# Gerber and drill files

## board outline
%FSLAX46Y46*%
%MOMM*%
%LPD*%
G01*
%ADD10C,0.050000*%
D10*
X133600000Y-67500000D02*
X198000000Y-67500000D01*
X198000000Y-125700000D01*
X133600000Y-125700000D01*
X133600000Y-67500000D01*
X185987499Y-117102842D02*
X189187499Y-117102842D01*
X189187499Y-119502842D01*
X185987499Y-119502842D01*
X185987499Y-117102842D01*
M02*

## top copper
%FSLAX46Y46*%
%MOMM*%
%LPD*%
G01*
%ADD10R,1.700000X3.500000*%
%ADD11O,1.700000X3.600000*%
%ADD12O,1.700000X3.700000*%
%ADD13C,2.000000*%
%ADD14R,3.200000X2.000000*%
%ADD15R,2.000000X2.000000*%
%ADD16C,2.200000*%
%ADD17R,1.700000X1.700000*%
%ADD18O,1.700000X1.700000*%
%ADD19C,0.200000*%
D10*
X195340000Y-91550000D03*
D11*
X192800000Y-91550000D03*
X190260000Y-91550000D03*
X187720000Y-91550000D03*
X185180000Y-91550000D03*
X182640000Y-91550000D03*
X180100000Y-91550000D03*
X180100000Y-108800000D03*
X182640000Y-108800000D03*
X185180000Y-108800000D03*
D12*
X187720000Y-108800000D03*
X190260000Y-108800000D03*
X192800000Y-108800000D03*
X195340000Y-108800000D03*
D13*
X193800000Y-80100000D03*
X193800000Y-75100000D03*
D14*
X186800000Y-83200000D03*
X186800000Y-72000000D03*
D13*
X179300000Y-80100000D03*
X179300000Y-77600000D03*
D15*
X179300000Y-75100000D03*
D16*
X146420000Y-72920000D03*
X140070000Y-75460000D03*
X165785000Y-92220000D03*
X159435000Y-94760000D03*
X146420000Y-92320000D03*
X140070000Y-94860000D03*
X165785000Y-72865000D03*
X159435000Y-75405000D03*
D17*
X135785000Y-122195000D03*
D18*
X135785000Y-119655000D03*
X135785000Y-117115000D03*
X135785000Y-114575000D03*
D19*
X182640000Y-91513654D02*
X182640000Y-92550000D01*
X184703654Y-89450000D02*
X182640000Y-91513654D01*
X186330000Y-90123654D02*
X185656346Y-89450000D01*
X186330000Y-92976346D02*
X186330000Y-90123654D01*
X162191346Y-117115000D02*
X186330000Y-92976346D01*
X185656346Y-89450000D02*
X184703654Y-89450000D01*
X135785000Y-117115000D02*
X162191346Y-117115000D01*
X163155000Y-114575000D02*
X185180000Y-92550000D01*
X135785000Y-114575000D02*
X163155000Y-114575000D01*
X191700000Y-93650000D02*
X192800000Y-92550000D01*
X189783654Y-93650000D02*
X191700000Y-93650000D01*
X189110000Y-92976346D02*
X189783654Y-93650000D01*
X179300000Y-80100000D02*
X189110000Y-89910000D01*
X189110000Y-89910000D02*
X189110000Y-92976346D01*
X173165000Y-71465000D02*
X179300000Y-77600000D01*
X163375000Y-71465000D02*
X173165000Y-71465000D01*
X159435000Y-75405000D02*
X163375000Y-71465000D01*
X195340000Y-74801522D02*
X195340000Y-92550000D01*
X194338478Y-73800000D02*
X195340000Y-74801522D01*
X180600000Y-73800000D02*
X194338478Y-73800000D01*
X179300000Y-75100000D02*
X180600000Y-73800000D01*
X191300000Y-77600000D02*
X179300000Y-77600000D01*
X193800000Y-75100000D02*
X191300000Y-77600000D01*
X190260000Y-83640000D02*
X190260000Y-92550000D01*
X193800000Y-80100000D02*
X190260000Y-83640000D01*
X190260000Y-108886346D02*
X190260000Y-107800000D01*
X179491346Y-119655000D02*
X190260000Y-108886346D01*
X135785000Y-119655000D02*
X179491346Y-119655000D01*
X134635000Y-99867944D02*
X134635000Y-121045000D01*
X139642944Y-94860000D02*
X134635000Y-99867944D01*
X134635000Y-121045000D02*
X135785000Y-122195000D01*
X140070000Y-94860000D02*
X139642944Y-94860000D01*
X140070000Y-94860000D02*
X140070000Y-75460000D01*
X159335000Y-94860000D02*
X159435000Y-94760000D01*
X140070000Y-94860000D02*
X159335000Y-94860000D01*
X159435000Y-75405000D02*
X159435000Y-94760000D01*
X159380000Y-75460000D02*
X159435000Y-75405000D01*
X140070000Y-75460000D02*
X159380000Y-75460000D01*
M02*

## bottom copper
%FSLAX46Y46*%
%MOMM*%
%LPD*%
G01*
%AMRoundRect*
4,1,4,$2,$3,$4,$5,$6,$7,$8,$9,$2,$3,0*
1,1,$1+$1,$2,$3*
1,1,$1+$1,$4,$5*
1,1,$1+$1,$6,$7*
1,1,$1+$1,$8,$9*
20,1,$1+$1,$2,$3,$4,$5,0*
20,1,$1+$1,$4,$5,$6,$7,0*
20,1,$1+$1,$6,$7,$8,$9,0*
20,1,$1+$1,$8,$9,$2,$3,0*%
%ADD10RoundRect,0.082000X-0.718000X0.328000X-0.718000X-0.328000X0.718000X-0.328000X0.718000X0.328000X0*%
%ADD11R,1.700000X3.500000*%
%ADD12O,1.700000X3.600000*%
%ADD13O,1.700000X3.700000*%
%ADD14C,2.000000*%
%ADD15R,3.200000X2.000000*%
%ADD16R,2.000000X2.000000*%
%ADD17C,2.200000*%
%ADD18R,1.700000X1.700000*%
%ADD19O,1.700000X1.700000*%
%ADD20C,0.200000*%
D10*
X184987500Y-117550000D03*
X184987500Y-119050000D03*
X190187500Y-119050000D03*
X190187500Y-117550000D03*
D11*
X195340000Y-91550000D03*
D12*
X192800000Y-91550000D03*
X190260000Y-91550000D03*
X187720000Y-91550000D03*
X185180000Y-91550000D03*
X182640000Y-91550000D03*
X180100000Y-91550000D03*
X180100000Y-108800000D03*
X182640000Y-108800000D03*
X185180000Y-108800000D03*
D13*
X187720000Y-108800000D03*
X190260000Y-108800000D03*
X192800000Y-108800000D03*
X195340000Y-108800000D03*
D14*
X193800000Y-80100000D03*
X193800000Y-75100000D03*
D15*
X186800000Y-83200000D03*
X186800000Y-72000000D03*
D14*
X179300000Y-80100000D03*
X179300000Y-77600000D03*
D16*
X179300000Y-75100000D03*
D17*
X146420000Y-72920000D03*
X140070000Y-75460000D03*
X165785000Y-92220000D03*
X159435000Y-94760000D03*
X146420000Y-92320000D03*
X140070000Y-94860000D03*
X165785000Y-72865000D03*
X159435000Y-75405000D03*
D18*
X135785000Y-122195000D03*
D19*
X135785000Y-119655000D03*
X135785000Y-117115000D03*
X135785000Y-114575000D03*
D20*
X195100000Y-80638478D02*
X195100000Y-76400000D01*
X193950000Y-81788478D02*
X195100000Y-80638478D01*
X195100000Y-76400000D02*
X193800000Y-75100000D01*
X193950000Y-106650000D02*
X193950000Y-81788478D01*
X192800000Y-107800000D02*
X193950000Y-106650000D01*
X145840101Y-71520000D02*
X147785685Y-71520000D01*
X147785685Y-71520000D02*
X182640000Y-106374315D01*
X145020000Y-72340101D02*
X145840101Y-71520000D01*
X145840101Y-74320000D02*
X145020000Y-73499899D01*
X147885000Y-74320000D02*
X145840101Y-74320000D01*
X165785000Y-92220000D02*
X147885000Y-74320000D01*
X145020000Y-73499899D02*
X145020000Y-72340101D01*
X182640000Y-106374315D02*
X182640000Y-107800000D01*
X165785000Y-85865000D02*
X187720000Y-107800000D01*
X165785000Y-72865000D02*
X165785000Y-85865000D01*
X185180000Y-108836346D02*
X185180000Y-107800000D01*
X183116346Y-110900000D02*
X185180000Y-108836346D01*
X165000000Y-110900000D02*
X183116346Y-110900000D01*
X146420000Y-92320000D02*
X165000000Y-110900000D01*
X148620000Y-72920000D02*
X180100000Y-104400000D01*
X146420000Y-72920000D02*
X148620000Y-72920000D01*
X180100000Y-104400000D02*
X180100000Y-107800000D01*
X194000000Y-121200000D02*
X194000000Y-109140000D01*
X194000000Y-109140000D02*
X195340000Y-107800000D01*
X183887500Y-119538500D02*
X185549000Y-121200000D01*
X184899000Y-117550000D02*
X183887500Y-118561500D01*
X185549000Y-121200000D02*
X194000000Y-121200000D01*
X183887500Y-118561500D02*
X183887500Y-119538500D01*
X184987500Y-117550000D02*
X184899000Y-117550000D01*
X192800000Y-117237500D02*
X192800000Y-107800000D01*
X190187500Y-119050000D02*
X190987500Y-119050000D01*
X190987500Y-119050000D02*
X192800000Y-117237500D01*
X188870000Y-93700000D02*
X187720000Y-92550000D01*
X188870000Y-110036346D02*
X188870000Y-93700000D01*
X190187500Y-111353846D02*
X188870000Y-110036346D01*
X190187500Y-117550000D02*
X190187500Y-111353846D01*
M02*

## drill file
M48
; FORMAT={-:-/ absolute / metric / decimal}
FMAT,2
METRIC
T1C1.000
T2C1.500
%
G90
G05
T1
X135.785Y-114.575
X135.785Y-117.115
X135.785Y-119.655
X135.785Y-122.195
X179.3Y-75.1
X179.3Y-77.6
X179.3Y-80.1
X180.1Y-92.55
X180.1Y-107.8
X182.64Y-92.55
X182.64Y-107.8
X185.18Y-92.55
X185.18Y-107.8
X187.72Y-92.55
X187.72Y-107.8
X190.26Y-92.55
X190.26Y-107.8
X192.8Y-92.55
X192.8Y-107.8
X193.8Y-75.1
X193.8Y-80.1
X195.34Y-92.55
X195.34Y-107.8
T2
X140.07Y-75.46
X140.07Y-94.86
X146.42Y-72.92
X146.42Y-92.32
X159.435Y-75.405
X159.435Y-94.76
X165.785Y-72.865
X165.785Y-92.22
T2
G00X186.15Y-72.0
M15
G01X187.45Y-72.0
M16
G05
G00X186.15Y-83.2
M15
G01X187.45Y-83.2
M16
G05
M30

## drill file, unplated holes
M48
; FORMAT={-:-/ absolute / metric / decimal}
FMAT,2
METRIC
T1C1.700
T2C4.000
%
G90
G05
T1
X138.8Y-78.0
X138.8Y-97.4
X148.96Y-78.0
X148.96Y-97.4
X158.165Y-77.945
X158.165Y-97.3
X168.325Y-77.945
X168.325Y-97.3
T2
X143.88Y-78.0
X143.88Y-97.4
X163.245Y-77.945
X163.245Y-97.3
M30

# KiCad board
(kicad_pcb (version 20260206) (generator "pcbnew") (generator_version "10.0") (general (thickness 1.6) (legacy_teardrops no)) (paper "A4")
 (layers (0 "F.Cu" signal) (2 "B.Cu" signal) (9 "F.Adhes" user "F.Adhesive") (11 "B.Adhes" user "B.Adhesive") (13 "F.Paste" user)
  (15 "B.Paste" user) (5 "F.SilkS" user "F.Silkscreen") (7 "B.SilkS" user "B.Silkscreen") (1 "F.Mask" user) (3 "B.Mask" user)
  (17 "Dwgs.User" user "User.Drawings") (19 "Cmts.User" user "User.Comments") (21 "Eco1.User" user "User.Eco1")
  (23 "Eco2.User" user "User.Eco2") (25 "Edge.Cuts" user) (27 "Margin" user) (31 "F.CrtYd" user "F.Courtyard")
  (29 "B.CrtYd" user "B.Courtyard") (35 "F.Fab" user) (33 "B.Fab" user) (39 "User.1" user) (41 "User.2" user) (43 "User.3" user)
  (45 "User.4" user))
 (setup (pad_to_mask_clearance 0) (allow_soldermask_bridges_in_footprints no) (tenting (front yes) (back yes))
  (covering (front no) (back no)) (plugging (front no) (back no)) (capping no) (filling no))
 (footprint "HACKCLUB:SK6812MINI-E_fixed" (layer "F.Cu") (at 187.587499 118.402842)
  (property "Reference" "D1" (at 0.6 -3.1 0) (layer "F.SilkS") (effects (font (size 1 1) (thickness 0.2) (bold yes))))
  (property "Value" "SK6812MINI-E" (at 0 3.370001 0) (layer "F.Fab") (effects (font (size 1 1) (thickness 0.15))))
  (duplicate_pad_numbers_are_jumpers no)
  (fp_rect (start -1.6 -1.3) (end 1.6 1.1) (stroke (width 0.05) (type default)) (fill no) (layer "Edge.Cuts"))
  (pad "1" smd roundrect (at -2.599999 -0.852842 270) (size 0.82 1.6) (layers "B.Cu" "B.Mask" "B.Paste") (roundrect_rratio 0.1)
   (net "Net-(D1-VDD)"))
  (pad "2" smd roundrect (at -2.599999 0.647158 270) (size 0.82 1.6) (layers "B.Cu" "B.Mask" "B.Paste") (roundrect_rratio 0.1)
   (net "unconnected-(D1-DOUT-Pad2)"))
  (pad "3" smd roundrect (at 2.600001 0.647158 270) (size 0.82 1.6) (layers "B.Cu" "B.Mask" "B.Paste") (roundrect_rratio 0.1) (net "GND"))
  (pad "4" smd roundrect (at 2.600001 -0.852842 270) (size 0.82 1.6) (layers "B.Cu" "B.Mask" "B.Paste") (roundrect_rratio 0.1)
   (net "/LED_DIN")))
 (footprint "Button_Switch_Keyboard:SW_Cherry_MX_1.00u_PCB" (layer "F.Cu") (at 165.785 72.865)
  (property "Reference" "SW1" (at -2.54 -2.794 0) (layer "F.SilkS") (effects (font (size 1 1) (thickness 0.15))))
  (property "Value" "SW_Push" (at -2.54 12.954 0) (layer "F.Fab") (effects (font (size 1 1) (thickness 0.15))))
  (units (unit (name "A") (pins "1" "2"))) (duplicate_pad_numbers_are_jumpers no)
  (pad "" np_thru_hole circle (at -7.62 5.08) (size 1.7 1.7) (drill 1.7) (layers "*.Cu" "*.Mask"))
  (pad "" np_thru_hole circle (at -2.54 5.08) (size 4 4) (drill 4) (layers "*.Cu" "*.Mask"))
  (pad "" np_thru_hole circle (at 2.54 5.08) (size 1.7 1.7) (drill 1.7) (layers "*.Cu" "*.Mask"))
  (pad "1" thru_hole circle (at 0 0) (size 2.2 2.2) (drill 1.5) (layers "*.Cu" "*.Mask") (remove_unused_layers no)
   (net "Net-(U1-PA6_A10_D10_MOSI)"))
  (pad "2" thru_hole circle (at -6.35 2.54) (size 2.2 2.2) (drill 1.5) (layers "*.Cu" "*.Mask") (remove_unused_layers no) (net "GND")))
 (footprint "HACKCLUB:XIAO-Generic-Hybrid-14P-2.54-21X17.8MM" (layer "F.Cu") (at 187.72 100.175 -90)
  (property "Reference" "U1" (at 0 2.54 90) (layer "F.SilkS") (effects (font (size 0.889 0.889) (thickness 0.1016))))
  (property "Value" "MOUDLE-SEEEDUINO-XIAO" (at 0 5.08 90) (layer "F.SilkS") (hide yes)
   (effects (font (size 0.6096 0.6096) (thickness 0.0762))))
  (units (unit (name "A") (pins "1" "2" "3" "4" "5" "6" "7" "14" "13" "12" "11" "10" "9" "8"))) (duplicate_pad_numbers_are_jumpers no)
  (pad "1" thru_hole rect (at -7.625 -7.62 270) (size 3.5 1.7) (drill 1 (offset -1 0)) (layers "*.Cu" "*.Mask") (remove_unused_layers no)
   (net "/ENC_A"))
  (pad "2" thru_hole oval (at -7.625 -5.08 270) (size 3.6 1.7) (drill 1 (offset -1 0)) (layers "*.Cu" "*.Mask") (remove_unused_layers no)
   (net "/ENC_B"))
  (pad "3" thru_hole oval (at -7.625 -2.54 270) (size 3.6 1.7) (drill 1 (offset -1 0)) (layers "*.Cu" "*.Mask") (remove_unused_layers no)
   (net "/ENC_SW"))
  (pad "4" thru_hole oval (at -7.625 0 270) (size 3.6 1.7) (drill 1 (offset -1 0)) (layers "*.Cu" "*.Mask") (remove_unused_layers no)
   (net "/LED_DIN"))
  (pad "5" thru_hole oval (at -7.625 2.54 270) (size 3.6 1.7) (drill 1 (offset -1 0)) (layers "*.Cu" "*.Mask") (remove_unused_layers no)
   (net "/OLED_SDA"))
  (pad "6" thru_hole oval (at -7.625 5.08 90) (size 3.6 1.7) (drill 1 (offset 1 0)) (layers "*.Cu" "*.Mask") (remove_unused_layers no)
   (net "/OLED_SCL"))
  (pad "7" thru_hole oval (at -7.625 7.62 270) (size 3.6 1.7) (drill 1 (offset -1 0)) (layers "*.Cu" "*.Mask") (remove_unused_layers no)
   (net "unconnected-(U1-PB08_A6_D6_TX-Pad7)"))
  (pad "8" thru_hole oval (at 7.625 7.62 270) (size 3.6 1.7) (drill 1 (offset 1 0)) (layers "*.Cu" "*.Mask") (remove_unused_layers no)
   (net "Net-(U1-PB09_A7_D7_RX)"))
  (pad "9" thru_hole oval (at 7.625 5.08 270) (size 3.6 1.7) (drill 1 (offset 1 0)) (layers "*.Cu" "*.Mask") (remove_unused_layers no)
   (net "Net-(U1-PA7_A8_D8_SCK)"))
  (pad "10" thru_hole oval (at 7.625 2.54 270) (size 3.6 1.7) (drill 1 (offset 1 0)) (layers "*.Cu" "*.Mask") (remove_unused_layers no)
   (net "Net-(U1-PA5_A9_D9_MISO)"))
  (pad "11" thru_hole oval (at 7.625 0 270) (size 3.7 1.7) (drill 1 (offset 1 0)) (layers "*.Cu" "*.Mask") (remove_unused_layers no)
   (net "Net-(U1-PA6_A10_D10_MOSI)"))
  (pad "12" thru_hole oval (at 7.625 -2.54 270) (size 3.7 1.7) (drill 1 (offset 1 0)) (layers "*.Cu" "*.Mask") (remove_unused_layers no)
   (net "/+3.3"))
  (pad "13" thru_hole oval (at 7.625 -5.08 270) (size 3.7 1.7) (drill 1 (offset 1 0)) (layers "*.Cu" "*.Mask") (remove_unused_layers no)
   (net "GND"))
  (pad "14" thru_hole oval (at 7.625 -7.62 270) (size 3.7 1.7) (drill 1 (offset 1 0)) (layers "*.Cu" "*.Mask") (remove_unused_layers no)
   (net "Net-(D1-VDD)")))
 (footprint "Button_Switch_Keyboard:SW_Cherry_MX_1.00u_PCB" (layer "F.Cu") (at 146.42 92.32)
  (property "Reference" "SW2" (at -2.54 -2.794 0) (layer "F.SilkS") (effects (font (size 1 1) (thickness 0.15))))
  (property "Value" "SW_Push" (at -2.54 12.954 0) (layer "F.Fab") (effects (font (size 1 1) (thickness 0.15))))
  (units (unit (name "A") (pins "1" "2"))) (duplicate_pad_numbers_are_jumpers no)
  (pad "" np_thru_hole circle (at -7.62 5.08) (size 1.7 1.7) (drill 1.7) (layers "*.Cu" "*.Mask"))
  (pad "" np_thru_hole circle (at -2.54 5.08) (size 4 4) (drill 4) (layers "*.Cu" "*.Mask"))
  (pad "" np_thru_hole circle (at 2.54 5.08) (size 1.7 1.7) (drill 1.7) (layers "*.Cu" "*.Mask"))
  (pad "1" thru_hole circle (at 0 0) (size 2.2 2.2) (drill 1.5) (layers "*.Cu" "*.Mask") (remove_unused_layers no)
   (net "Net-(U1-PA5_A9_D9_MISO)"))
  (pad "2" thru_hole circle (at -6.35 2.54) (size 2.2 2.2) (drill 1.5) (layers "*.Cu" "*.Mask") (remove_unused_layers no) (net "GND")))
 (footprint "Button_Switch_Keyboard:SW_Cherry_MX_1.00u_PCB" (layer "F.Cu") (at 146.42 72.92)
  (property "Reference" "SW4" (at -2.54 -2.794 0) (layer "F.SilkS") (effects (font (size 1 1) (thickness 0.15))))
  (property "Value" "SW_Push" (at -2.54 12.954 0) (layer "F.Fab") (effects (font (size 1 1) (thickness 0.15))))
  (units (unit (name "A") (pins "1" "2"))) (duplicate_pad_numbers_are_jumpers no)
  (pad "" np_thru_hole circle (at -7.62 5.08) (size 1.7 1.7) (drill 1.7) (layers "*.Cu" "*.Mask"))
  (pad "" np_thru_hole circle (at -2.54 5.08) (size 4 4) (drill 4) (layers "*.Cu" "*.Mask"))
  (pad "" np_thru_hole circle (at 2.54 5.08) (size 1.7 1.7) (drill 1.7) (layers "*.Cu" "*.Mask"))
  (pad "1" thru_hole circle (at 0 0) (size 2.2 2.2) (drill 1.5) (layers "*.Cu" "*.Mask") (remove_unused_layers no)
   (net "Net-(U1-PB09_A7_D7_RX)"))
  (pad "2" thru_hole circle (at -6.35 2.54) (size 2.2 2.2) (drill 1.5) (layers "*.Cu" "*.Mask") (remove_unused_layers no) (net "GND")))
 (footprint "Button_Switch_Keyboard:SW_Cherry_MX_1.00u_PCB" (layer "F.Cu") (at 165.785 92.22)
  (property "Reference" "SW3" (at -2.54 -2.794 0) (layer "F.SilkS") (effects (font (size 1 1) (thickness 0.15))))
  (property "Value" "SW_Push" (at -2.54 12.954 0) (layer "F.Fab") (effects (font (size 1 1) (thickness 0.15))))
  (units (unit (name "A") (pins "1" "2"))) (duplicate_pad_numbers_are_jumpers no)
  (pad "" np_thru_hole circle (at -7.62 5.08) (size 1.7 1.7) (drill 1.7) (layers "*.Cu" "*.Mask"))
  (pad "" np_thru_hole circle (at -2.54 5.08) (size 4 4) (drill 4) (layers "*.Cu" "*.Mask"))
  (pad "" np_thru_hole circle (at 2.54 5.08) (size 1.7 1.7) (drill 1.7) (layers "*.Cu" "*.Mask"))
  (pad "1" thru_hole circle (at 0 0) (size 2.2 2.2) (drill 1.5) (layers "*.Cu" "*.Mask") (remove_unused_layers no)
   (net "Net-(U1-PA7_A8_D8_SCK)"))
  (pad "2" thru_hole circle (at -6.35 2.54) (size 2.2 2.2) (drill 1.5) (layers "*.Cu" "*.Mask") (remove_unused_layers no) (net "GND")))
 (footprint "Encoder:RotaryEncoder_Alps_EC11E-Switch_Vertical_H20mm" (layer "F.Cu") (at 179.3 75.1)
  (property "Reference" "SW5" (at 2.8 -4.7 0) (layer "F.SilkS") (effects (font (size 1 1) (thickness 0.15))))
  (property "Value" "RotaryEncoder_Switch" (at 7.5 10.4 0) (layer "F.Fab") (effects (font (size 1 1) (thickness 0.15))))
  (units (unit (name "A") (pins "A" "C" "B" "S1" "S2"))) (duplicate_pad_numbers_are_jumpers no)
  (pad "A" thru_hole rect (at 0 0) (size 2 2) (drill 1) (layers "*.Cu" "*.Mask") (remove_unused_layers no) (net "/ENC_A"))
  (pad "B" thru_hole circle (at 0 5) (size 2 2) (drill 1) (layers "*.Cu" "*.Mask") (remove_unused_layers no) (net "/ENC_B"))
  (pad "C" thru_hole circle (at 0 2.5) (size 2 2) (drill 1) (layers "*.Cu" "*.Mask") (remove_unused_layers no) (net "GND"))
  (pad "MP" thru_hole rect (at 7.5 -3.1) (size 3.2 2) (drill oval 2.8 1.5) (layers "*.Cu" "*.Mask") (remove_unused_layers no))
  (pad "MP" thru_hole rect (at 7.5 8.1) (size 3.2 2) (drill oval 2.8 1.5) (layers "*.Cu" "*.Mask") (remove_unused_layers no))
  (pad "S1" thru_hole circle (at 14.5 5) (size 2 2) (drill 1) (layers "*.Cu" "*.Mask") (remove_unused_layers no) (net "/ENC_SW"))
  (pad "S2" thru_hole circle (at 14.5 0) (size 2 2) (drill 1) (layers "*.Cu" "*.Mask") (remove_unused_layers no) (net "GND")))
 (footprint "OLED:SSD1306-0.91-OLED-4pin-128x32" (layer "F.Cu") (at 172.285 124.385 180)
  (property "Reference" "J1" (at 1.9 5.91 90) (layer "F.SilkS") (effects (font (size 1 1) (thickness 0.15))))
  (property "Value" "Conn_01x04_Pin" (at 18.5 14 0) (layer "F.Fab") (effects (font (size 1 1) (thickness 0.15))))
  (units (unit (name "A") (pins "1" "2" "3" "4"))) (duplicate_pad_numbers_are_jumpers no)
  (pad "1" thru_hole rect (at 36.5 2.19 180) (size 1.7 1.7) (drill 1) (layers "*.Cu" "*.Mask") (remove_unused_layers no) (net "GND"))
  (pad "2" thru_hole oval (at 36.5 4.73 180) (size 1.7 1.7) (drill 1) (layers "*.Cu" "*.Mask") (remove_unused_layers no) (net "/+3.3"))
  (pad "3" thru_hole oval (at 36.5 7.27 180) (size 1.7 1.7) (drill 1) (layers "*.Cu" "*.Mask") (remove_unused_layers no) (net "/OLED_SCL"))
  (pad "4" thru_hole oval (at 36.5 9.81 180) (size 1.7 1.7) (drill 1) (layers "*.Cu" "*.Mask") (remove_unused_layers no) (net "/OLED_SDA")))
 (gr_rect (start 133.6 67.5) (end 198 125.7) (stroke (width 0.05) (type default)) (fill no) (layer "Edge.Cuts"))
 (segment (start 165.785 72.865) (end 165.785 85.865) (width 0.2) (layer "B.Cu") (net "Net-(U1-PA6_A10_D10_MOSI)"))
 (segment (start 165.785 85.865) (end 187.72 107.8) (width 0.2) (layer "B.Cu") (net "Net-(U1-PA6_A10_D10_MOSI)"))
 (segment (start 140.07 94.86) (end 159.335 94.86) (width 0.2) (layer "F.Cu") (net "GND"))
 (segment (start 159.38 75.46) (end 159.435 75.405) (width 0.2) (layer "F.Cu") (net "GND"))
 (segment (start 134.635 99.867944) (end 134.635 121.045) (width 0.2) (layer "F.Cu") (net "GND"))
 (segment (start 191.3 77.6) (end 179.3 77.6) (width 0.2) (layer "F.Cu") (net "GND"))
 (segment (start 159.335 94.86) (end 159.435 94.76) (width 0.2) (layer "F.Cu") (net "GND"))
 (segment (start 159.435 75.405) (end 163.375 71.465) (width 0.2) (layer "F.Cu") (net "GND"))
 (segment (start 159.435 75.405) (end 159.435 94.76) (width 0.2) (layer "F.Cu") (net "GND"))
 (segment (start 163.375 71.465) (end 173.165 71.465) (width 0.2) (layer "F.Cu") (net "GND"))
 (segment (start 140.07 75.46) (end 159.38 75.46) (width 0.2) (layer "F.Cu") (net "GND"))
 (segment (start 173.165 71.465) (end 179.3 77.6) (width 0.2) (layer "F.Cu") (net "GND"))
 (segment (start 193.8 75.1) (end 191.3 77.6) (width 0.2) (layer "F.Cu") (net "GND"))
 (segment (start 140.07 94.86) (end 139.642944 94.86) (width 0.2) (layer "F.Cu") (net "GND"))
 (segment (start 139.642944 94.86) (end 134.635 99.867944) (width 0.2) (layer "F.Cu") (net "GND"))
 (segment (start 140.07 94.86) (end 140.07 75.46) (width 0.2) (layer "F.Cu") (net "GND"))
 (segment (start 134.635 121.045) (end 135.785 122.195) (width 0.2) (layer "F.Cu") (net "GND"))
 (segment (start 193.95 81.788478) (end 195.1 80.638478) (width 0.2) (layer "B.Cu") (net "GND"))
 (segment (start 192.8 107.8) (end 193.95 106.65) (width 0.2) (layer "B.Cu") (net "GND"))
 (segment (start 190.9875 119.05) (end 192.8 117.2375) (width 0.2) (layer "B.Cu") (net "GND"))
 (segment (start 195.1 76.4) (end 193.8 75.1) (width 0.2) (layer "B.Cu") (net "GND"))
 (segment (start 193.95 106.65) (end 193.95 81.788478) (width 0.2) (layer "B.Cu") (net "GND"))
 (segment (start 192.8 117.2375) (end 192.8 107.8) (width 0.2) (layer "B.Cu") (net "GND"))
 (segment (start 190.1875 119.05) (end 190.9875 119.05) (width 0.2) (layer "B.Cu") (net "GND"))
 (segment (start 195.1 80.638478) (end 195.1 76.4) (width 0.2) (layer "B.Cu") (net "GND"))
 (segment (start 195.34 74.801522) (end 195.34 92.55) (width 0.2) (layer "F.Cu") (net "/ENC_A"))
 (segment (start 194.338478 73.8) (end 195.34 74.801522) (width 0.2) (layer "F.Cu") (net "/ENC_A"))
 (segment (start 179.3 75.1) (end 180.6 73.8) (width 0.2) (layer "F.Cu") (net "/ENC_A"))
 (segment (start 180.6 73.8) (end 194.338478 73.8) (width 0.2) (layer "F.Cu") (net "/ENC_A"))
 (segment (start 189.783654 93.65) (end 191.7 93.65) (width 0.2) (layer "F.Cu") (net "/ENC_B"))
 (segment (start 179.3 80.1) (end 189.11 89.91) (width 0.2) (layer "F.Cu") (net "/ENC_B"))
 (segment (start 189.11 89.91) (end 189.11 92.976346) (width 0.2) (layer "F.Cu") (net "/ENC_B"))
 (segment (start 189.11 92.976346) (end 189.783654 93.65) (width 0.2) (layer "F.Cu") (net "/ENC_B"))
 (segment (start 191.7 93.65) (end 192.8 92.55) (width 0.2) (layer "F.Cu") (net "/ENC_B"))
 (segment (start 190.26 83.64) (end 190.26 92.55) (width 0.2) (layer "F.Cu") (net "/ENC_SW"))
 (segment (start 193.8 80.1) (end 190.26 83.64) (width 0.2) (layer "F.Cu") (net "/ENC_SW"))
 (segment (start 182.64 106.374315) (end 182.64 107.8) (width 0.2) (layer "B.Cu") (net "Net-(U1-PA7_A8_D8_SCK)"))
 (segment (start 147.885 74.32) (end 145.840101 74.32) (width 0.2) (layer "B.Cu") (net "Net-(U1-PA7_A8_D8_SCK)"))
 (segment (start 147.785685 71.52) (end 182.64 106.374315) (width 0.2) (layer "B.Cu") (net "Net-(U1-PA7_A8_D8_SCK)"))
 (segment (start 145.02 72.340101) (end 145.840101 71.52) (width 0.2) (layer "B.Cu") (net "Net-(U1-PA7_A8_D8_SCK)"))
 (segment (start 165.785 92.22) (end 147.885 74.32) (width 0.2) (layer "B.Cu") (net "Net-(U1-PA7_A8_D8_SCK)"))
 (segment (start 145.840101 71.52) (end 147.785685 71.52) (width 0.2) (layer "B.Cu") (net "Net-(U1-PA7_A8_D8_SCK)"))
 (segment (start 145.840101 74.32) (end 145.02 73.499899) (width 0.2) (layer "B.Cu") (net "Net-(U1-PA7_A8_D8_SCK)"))
 (segment (start 145.02 73.499899) (end 145.02 72.340101) (width 0.2) (layer "B.Cu") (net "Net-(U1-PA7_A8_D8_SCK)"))
 (segment (start 190.26 108.886346) (end 190.26 107.8) (width 0.2) (layer "F.Cu") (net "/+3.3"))
 (segment (start 135.785 119.655) (end 179.491346 119.655) (width 0.2) (layer "F.Cu") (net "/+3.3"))
 (segment (start 179.491346 119.655) (end 190.26 108.886346) (width 0.2) (layer "F.Cu") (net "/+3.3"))
 (segment (start 184.703654 89.45) (end 182.64 91.513654) (width 0.2) (layer "F.Cu") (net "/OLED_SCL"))
 (segment (start 182.64 91.513654) (end 182.64 92.55) (width 0.2) (layer "F.Cu") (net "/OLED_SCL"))
 (segment (start 186.33 92.976346) (end 186.33 90.123654) (width 0.2) (layer "F.Cu") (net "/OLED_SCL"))
 (segment (start 185.656346 89.45) (end 184.703654 89.45) (width 0.2) (layer "F.Cu") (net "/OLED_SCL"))
 (segment (start 135.785 117.115) (end 162.191346 117.115) (width 0.2) (layer "F.Cu") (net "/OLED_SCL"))
 (segment (start 162.191346 117.115) (end 186.33 92.976346) (width 0.2) (layer "F.Cu") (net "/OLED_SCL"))
 (segment (start 186.33 90.123654) (end 185.656346 89.45) (width 0.2) (layer "F.Cu") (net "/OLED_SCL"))
 (segment (start 163.155 114.575) (end 185.18 92.55) (width 0.2) (layer "F.Cu") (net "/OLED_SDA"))
 (segment (start 135.785 114.575) (end 163.155 114.575) (width 0.2) (layer "F.Cu") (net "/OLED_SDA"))
 (segment (start 185.18 108.836346) (end 185.18 107.8) (width 0.2) (layer "B.Cu") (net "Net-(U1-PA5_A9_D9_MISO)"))
 (segment (start 146.42 92.32) (end 165 110.9) (width 0.2) (layer "B.Cu") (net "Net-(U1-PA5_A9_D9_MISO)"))
 (segment (start 165 110.9) (end 183.116346 110.9) (width 0.2) (layer "B.Cu") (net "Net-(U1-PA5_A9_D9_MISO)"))
 (segment (start 183.116346 110.9) (end 185.18 108.836346) (width 0.2) (layer "B.Cu") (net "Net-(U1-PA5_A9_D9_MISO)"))
 (segment (start 146.42 72.92) (end 148.62 72.92) (width 0.2) (layer "B.Cu") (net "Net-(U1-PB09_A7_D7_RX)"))
 (segment (start 180.1 104.4) (end 180.1 107.8) (width 0.2) (layer "B.Cu") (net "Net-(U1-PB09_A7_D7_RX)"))
 (segment (start 148.62 72.92) (end 180.1 104.4) (width 0.2) (layer "B.Cu") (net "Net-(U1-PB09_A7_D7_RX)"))
 (segment (start 184.899 117.55) (end 183.8875 118.5615) (width 0.2) (layer "B.Cu") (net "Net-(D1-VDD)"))
 (segment (start 183.8875 119.5385) (end 185.549 121.2) (width 0.2) (layer "B.Cu") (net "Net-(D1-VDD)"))
 (segment (start 194 109.14) (end 195.34 107.8) (width 0.2) (layer "B.Cu") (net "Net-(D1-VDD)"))
 (segment (start 194 121.2) (end 194 109.14) (width 0.2) (layer "B.Cu") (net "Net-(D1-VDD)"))
 (segment (start 183.8875 118.5615) (end 183.8875 119.5385) (width 0.2) (layer "B.Cu") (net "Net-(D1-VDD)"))
 (segment (start 184.9875 117.55) (end 184.899 117.55) (width 0.2) (layer "B.Cu") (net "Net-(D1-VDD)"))
 (segment (start 185.549 121.2) (end 194 121.2) (width 0.2) (layer "B.Cu") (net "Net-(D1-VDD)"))
 (segment (start 188.87 110.036346) (end 188.87 93.7) (width 0.2) (layer "B.Cu") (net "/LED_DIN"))
 (segment (start 190.1875 111.353846) (end 188.87 110.036346) (width 0.2) (layer "B.Cu") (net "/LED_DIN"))
 (segment (start 190.1875 117.55) (end 190.1875 111.353846) (width 0.2) (layer "B.Cu") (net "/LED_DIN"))
 (segment (start 188.87 93.7) (end 187.72 92.55) (width 0.2) (layer "B.Cu") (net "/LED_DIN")))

